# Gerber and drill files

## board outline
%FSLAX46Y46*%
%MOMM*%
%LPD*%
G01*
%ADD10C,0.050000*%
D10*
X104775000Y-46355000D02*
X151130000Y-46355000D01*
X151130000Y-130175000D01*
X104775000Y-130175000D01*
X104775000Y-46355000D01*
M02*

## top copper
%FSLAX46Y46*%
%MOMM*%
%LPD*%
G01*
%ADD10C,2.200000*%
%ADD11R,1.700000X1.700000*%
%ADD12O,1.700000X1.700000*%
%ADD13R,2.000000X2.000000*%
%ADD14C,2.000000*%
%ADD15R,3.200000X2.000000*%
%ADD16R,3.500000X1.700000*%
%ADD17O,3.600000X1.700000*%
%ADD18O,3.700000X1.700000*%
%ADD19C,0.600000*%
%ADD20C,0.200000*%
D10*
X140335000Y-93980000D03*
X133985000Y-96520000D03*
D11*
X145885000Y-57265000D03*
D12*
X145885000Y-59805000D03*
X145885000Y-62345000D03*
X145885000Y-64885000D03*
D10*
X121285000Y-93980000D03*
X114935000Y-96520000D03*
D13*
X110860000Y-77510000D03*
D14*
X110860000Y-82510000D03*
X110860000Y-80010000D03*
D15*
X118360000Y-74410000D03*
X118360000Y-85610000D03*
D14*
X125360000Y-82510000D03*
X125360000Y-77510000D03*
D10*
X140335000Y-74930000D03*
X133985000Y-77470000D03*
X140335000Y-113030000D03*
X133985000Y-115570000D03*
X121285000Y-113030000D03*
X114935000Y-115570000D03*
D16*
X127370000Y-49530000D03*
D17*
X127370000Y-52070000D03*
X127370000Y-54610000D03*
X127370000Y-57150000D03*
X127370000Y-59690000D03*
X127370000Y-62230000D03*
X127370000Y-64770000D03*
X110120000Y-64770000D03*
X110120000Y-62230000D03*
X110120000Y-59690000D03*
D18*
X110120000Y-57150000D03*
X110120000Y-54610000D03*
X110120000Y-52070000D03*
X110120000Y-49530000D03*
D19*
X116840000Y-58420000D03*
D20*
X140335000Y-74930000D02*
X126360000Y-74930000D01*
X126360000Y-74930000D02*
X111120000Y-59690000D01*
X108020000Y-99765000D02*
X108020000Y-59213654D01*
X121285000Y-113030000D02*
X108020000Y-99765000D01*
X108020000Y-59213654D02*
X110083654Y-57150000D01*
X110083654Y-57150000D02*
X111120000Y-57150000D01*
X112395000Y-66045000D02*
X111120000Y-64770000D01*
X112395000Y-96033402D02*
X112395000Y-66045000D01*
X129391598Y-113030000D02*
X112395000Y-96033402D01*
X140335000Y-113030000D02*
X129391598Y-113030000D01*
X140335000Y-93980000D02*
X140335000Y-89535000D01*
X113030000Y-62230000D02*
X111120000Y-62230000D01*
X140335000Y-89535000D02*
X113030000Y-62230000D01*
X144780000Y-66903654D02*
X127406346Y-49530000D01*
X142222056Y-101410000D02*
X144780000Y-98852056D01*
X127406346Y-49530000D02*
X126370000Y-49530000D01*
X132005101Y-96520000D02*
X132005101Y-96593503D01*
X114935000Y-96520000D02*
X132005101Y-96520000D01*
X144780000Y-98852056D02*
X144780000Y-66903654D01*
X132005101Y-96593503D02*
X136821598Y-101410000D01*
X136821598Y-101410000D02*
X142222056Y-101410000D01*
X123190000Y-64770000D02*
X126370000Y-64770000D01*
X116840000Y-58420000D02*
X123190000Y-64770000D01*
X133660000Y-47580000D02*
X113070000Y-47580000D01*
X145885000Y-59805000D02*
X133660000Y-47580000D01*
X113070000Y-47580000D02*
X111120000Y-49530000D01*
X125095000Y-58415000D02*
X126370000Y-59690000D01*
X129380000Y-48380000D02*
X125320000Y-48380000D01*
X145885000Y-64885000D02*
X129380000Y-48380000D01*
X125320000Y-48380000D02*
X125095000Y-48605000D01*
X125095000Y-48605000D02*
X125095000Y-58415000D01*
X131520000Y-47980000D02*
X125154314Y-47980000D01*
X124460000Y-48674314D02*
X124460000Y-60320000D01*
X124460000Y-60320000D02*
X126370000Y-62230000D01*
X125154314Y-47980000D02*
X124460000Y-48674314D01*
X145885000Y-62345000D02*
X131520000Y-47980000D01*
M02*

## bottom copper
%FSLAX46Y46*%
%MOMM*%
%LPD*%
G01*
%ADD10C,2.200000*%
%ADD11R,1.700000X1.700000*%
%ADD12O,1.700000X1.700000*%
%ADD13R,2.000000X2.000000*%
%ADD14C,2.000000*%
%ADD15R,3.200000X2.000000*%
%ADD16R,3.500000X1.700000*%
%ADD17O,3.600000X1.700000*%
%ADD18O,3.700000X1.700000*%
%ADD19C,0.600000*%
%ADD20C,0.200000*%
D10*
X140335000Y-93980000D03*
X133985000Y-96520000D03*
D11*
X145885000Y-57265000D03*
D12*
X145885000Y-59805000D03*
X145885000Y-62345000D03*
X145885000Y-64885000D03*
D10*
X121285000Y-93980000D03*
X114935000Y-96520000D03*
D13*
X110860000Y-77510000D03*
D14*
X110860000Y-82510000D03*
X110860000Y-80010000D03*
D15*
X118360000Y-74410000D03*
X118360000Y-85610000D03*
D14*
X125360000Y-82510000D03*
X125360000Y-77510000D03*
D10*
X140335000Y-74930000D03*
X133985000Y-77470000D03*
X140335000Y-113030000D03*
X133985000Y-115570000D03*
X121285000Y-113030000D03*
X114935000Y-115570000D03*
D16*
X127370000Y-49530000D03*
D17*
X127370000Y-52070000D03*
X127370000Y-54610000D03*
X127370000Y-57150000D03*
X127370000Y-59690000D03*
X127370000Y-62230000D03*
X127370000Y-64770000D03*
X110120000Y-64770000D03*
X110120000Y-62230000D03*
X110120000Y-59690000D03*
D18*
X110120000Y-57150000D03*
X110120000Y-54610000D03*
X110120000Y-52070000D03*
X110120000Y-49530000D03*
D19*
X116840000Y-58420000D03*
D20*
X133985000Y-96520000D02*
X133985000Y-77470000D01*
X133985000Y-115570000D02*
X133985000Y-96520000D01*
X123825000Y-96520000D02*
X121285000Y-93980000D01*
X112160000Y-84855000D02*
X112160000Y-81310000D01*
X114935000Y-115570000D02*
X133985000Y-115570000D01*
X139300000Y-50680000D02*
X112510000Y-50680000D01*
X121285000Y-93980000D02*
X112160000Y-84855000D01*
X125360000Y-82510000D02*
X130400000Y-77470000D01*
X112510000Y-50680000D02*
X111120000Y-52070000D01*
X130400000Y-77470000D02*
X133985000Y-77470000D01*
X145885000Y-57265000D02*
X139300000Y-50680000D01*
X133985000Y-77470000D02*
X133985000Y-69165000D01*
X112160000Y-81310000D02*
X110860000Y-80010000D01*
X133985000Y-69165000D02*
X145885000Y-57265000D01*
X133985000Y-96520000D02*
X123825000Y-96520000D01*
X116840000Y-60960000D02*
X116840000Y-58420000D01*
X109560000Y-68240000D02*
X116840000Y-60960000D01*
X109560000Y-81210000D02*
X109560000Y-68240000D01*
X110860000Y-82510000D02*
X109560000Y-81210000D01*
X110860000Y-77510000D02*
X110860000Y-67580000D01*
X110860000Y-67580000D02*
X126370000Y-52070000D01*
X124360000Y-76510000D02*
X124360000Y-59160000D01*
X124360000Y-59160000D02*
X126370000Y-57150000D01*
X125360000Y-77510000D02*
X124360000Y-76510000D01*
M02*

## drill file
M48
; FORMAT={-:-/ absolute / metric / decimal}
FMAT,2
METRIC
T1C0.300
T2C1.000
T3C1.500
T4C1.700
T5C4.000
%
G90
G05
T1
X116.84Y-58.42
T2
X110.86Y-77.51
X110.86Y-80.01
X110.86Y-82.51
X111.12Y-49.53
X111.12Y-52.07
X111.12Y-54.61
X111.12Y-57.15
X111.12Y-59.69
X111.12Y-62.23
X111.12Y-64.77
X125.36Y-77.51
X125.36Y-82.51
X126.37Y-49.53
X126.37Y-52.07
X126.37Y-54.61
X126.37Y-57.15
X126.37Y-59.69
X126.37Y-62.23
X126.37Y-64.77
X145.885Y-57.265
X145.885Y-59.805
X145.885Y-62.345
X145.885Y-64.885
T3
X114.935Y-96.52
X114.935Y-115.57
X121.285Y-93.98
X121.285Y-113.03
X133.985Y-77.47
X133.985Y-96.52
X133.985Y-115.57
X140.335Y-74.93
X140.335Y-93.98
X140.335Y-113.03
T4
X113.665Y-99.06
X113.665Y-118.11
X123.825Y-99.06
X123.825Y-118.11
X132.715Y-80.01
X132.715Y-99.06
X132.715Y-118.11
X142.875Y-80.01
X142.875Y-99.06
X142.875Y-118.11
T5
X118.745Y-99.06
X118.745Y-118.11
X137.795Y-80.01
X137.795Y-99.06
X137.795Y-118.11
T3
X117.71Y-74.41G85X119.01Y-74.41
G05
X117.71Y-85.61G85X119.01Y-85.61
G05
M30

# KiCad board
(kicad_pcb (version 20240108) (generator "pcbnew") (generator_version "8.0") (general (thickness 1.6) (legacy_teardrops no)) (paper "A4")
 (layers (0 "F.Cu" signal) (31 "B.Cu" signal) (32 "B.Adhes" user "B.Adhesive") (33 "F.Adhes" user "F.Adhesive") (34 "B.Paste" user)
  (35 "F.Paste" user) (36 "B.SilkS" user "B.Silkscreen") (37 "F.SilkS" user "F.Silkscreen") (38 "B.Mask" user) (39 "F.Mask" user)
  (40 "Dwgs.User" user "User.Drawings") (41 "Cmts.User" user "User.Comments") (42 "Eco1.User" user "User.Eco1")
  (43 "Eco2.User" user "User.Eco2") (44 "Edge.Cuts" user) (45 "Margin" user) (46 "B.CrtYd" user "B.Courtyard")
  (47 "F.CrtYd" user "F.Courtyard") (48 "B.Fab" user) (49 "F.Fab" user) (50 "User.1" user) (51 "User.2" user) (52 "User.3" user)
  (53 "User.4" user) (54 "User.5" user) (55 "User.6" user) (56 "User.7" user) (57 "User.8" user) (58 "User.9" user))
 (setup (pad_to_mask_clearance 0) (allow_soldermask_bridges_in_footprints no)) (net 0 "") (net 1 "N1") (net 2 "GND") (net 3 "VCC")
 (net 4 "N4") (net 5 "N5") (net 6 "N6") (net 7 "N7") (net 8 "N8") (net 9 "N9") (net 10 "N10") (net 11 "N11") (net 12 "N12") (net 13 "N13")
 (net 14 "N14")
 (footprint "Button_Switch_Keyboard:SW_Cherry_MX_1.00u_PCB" (layer "F.Cu") (at 140.335 93.98)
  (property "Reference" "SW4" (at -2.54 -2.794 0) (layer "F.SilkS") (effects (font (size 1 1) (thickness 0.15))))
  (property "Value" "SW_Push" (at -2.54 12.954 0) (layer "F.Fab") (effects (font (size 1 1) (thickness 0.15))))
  (pad "" np_thru_hole circle (at -7.62 5.08) (size 1.7 1.7) (drill 1.7) (layers "*.Cu" "*.Mask"))
  (pad "" np_thru_hole circle (at -2.54 5.08) (size 4 4) (drill 4) (layers "*.Cu" "*.Mask"))
  (pad "" np_thru_hole circle (at 2.54 5.08) (size 1.7 1.7) (drill 1.7) (layers "*.Cu" "*.Mask"))
  (pad "1" thru_hole circle (at 0 0) (size 2.2 2.2) (drill 1.5) (layers "*.Cu" "*.Mask") (remove_unused_layers no) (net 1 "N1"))
  (pad "2" thru_hole circle (at -6.35 2.54) (size 2.2 2.2) (drill 1.5) (layers "*.Cu" "*.Mask") (remove_unused_layers no) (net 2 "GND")))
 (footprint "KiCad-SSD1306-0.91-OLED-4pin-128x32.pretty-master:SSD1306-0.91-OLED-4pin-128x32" (layer "F.Cu") (at 109.385 55.075)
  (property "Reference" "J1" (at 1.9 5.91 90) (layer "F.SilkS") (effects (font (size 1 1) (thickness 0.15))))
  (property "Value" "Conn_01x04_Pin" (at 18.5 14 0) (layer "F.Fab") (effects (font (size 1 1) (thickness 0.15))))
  (pad "1" thru_hole rect (at 36.5 2.19) (size 1.7 1.7) (drill 1) (layers "*.Cu" "*.Mask") (remove_unused_layers no) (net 2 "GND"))
  (pad "2" thru_hole oval (at 36.5 4.73) (size 1.7 1.7) (drill 1) (layers "*.Cu" "*.Mask") (remove_unused_layers no) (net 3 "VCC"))
  (pad "3" thru_hole oval (at 36.5 7.27) (size 1.7 1.7) (drill 1) (layers "*.Cu" "*.Mask") (remove_unused_layers no) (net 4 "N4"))
  (pad "4" thru_hole oval (at 36.5 9.81) (size 1.7 1.7) (drill 1) (layers "*.Cu" "*.Mask") (remove_unused_layers no) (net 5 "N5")))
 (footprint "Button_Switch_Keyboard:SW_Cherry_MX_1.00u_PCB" (layer "F.Cu") (at 121.285 93.98)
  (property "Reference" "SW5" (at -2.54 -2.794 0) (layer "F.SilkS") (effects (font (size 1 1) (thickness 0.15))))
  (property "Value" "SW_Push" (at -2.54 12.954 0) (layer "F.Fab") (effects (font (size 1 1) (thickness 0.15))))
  (pad "" np_thru_hole circle (at -7.62 5.08) (size 1.7 1.7) (drill 1.7) (layers "*.Cu" "*.Mask"))
  (pad "" np_thru_hole circle (at -2.54 5.08) (size 4 4) (drill 4) (layers "*.Cu" "*.Mask"))
  (pad "" np_thru_hole circle (at 2.54 5.08) (size 1.7 1.7) (drill 1.7) (layers "*.Cu" "*.Mask"))
  (pad "1" thru_hole circle (at 0 0) (size 2.2 2.2) (drill 1.5) (layers "*.Cu" "*.Mask") (remove_unused_layers no) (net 2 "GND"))
  (pad "2" thru_hole circle (at -6.35 2.54) (size 2.2 2.2) (drill 1.5) (layers "*.Cu" "*.Mask") (remove_unused_layers no) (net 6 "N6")))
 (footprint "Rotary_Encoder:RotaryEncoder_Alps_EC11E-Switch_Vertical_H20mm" (layer "F.Cu") (at 110.86 77.51)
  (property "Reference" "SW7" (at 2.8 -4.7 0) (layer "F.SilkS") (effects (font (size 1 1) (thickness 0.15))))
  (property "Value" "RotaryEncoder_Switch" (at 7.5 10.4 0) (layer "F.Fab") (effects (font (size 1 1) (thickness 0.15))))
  (pad "A" thru_hole rect (at 0 0) (size 2 2) (drill 1) (layers "*.Cu" "*.Mask") (remove_unused_layers no) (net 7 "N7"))
  (pad "B" thru_hole circle (at 0 5) (size 2 2) (drill 1) (layers "*.Cu" "*.Mask") (remove_unused_layers no) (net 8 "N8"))
  (pad "C" thru_hole circle (at 0 2.5) (size 2 2) (drill 1) (layers "*.Cu" "*.Mask") (remove_unused_layers no) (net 2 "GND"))
  (pad "MP" thru_hole rect (at 7.5 -3.1) (size 3.2 2) (drill oval 2.8 1.5) (layers "*.Cu" "*.Mask") (remove_unused_layers no))
  (pad "MP" thru_hole rect (at 7.5 8.1) (size 3.2 2) (drill oval 2.8 1.5) (layers "*.Cu" "*.Mask") (remove_unused_layers no))
  (pad "S1" thru_hole circle (at 14.5 5) (size 2 2) (drill 1) (layers "*.Cu" "*.Mask") (remove_unused_layers no) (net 2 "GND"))
  (pad "S2" thru_hole circle (at 14.5 0) (size 2 2) (drill 1) (layers "*.Cu" "*.Mask") (remove_unused_layers no) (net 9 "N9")))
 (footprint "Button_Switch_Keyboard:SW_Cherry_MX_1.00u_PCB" (layer "F.Cu") (at 140.335 74.93)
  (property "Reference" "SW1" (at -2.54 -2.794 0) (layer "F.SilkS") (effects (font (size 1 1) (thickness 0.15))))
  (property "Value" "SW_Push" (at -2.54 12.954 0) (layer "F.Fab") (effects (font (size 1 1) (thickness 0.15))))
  (pad "" np_thru_hole circle (at -7.62 5.08) (size 1.7 1.7) (drill 1.7) (layers "*.Cu" "*.Mask"))
  (pad "" np_thru_hole circle (at -2.54 5.08) (size 4 4) (drill 4) (layers "*.Cu" "*.Mask"))
  (pad "" np_thru_hole circle (at 2.54 5.08) (size 1.7 1.7) (drill 1.7) (layers "*.Cu" "*.Mask"))
  (pad "1" thru_hole circle (at 0 0) (size 2.2 2.2) (drill 1.5) (layers "*.Cu" "*.Mask") (remove_unused_layers no) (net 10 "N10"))
  (pad "2" thru_hole circle (at -6.35 2.54) (size 2.2 2.2) (drill 1.5) (layers "*.Cu" "*.Mask") (remove_unused_layers no) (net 2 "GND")))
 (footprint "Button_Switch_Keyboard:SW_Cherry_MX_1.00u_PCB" (layer "F.Cu") (at 140.335 113.03)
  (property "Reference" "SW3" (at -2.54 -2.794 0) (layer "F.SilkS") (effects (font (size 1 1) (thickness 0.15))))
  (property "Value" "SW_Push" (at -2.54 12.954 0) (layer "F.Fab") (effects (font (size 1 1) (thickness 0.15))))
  (pad "" np_thru_hole circle (at -7.62 5.08) (size 1.7 1.7) (drill 1.7) (layers "*.Cu" "*.Mask"))
  (pad "" np_thru_hole circle (at -2.54 5.08) (size 4 4) (drill 4) (layers "*.Cu" "*.Mask"))
  (pad "" np_thru_hole circle (at 2.54 5.08) (size 1.7 1.7) (drill 1.7) (layers "*.Cu" "*.Mask"))
  (pad "1" thru_hole circle (at 0 0) (size 2.2 2.2) (drill 1.5) (layers "*.Cu" "*.Mask") (remove_unused_layers no) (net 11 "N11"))
  (pad "2" thru_hole circle (at -6.35 2.54) (size 2.2 2.2) (drill 1.5) (layers "*.Cu" "*.Mask") (remove_unused_layers no) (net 2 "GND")))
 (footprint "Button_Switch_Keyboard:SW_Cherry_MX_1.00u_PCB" (layer "F.Cu") (at 121.285 113.03)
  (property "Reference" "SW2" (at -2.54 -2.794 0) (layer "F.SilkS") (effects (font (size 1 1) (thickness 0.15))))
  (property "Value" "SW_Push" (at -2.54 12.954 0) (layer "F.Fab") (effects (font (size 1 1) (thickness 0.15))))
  (pad "" np_thru_hole circle (at -7.62 5.08) (size 1.7 1.7) (drill 1.7) (layers "*.Cu" "*.Mask"))
  (pad "" np_thru_hole circle (at -2.54 5.08) (size 4 4) (drill 4) (layers "*.Cu" "*.Mask"))
  (pad "" np_thru_hole circle (at 2.54 5.08) (size 1.7 1.7) (drill 1.7) (layers "*.Cu" "*.Mask"))
  (pad "1" thru_hole circle (at 0 0) (size 2.2 2.2) (drill 1.5) (layers "*.Cu" "*.Mask") (remove_unused_layers no) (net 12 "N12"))
  (pad "2" thru_hole circle (at -6.35 2.54) (size 2.2 2.2) (drill 1.5) (layers "*.Cu" "*.Mask") (remove_unused_layers no) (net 2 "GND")))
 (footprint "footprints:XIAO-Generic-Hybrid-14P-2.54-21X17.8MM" (layer "B.Cu") (at 118.745 57.15 180)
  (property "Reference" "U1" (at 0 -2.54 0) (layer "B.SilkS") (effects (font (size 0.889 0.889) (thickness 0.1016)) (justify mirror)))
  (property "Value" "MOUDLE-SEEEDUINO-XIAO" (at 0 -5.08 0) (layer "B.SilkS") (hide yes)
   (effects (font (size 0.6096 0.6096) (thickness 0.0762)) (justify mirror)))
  (pad "1" thru_hole rect (at -7.625 7.62 180) (size 3.5 1.7) (drill 1 (offset -1 0)) (layers "*.Cu" "*.Mask") (remove_unused_layers no)
   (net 6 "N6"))
  (pad "2" thru_hole oval (at -7.625 5.08 180) (size 3.6 1.7) (drill 1 (offset -1 0)) (layers "*.Cu" "*.Mask") (remove_unused_layers no)
   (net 7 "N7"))
  (pad "3" thru_hole oval (at -7.625 2.54 180) (size 3.6 1.7) (drill 1 (offset -1 0)) (layers "*.Cu" "*.Mask") (remove_unused_layers no)
   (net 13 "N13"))
  (pad "4" thru_hole oval (at -7.625 0 180) (size 3.6 1.7) (drill 1 (offset -1 0)) (layers "*.Cu" "*.Mask") (remove_unused_layers no)
   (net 9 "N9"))
  (pad "5" thru_hole oval (at -7.625 -2.54 180) (size 3.6 1.7) (drill 1 (offset -1 0)) (layers "*.Cu" "*.Mask") (remove_unused_layers no)
   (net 5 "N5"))
  (pad "6" thru_hole oval (at -7.625 -5.08) (size 3.6 1.7) (drill 1 (offset 1 0)) (layers "*.Cu" "*.Mask") (remove_unused_layers no)
   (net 4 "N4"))
  (pad "7" thru_hole oval (at -7.625 -7.62 180) (size 3.6 1.7) (drill 1 (offset -1 0)) (layers "*.Cu" "*.Mask") (remove_unused_layers no)
   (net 8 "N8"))
  (pad "8" thru_hole oval (at 7.625 -7.62 180) (size 3.6 1.7) (drill 1 (offset 1 0)) (layers "*.Cu" "*.Mask") (remove_unused_layers no)
   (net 11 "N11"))
  (pad "9" thru_hole oval (at 7.625 -5.08 180) (size 3.6 1.7) (drill 1 (offset 1 0)) (layers "*.Cu" "*.Mask") (remove_unused_layers no)
   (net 1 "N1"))
  (pad "10" thru_hole oval (at 7.625 -2.54 180) (size 3.6 1.7) (drill 1 (offset 1 0)) (layers "*.Cu" "*.Mask") (remove_unused_layers no)
   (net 10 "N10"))
  (pad "11" thru_hole oval (at 7.625 0 180) (size 3.7 1.7) (drill 1 (offset 1 0)) (layers "*.Cu" "*.Mask") (remove_unused_layers no)
   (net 12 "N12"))
  (pad "12" thru_hole oval (at 7.625 2.54 180) (size 3.7 1.7) (drill 1 (offset 1 0)) (layers "*.Cu" "*.Mask") (remove_unused_layers no)
   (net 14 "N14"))
  (pad "13" thru_hole oval (at 7.625 5.08 180) (size 3.7 1.7) (drill 1 (offset 1 0)) (layers "*.Cu" "*.Mask") (remove_unused_layers no)
   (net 2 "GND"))
  (pad "14" thru_hole oval (at 7.625 7.62 180) (size 3.7 1.7) (drill 1 (offset 1 0)) (layers "*.Cu" "*.Mask") (remove_unused_layers no)
   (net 3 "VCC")))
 (gr_rect (start 104.775 46.355) (end 151.13 130.175) (stroke (width 0.05) (type default)) (fill none) (layer "Edge.Cuts"))
 (segment (start 133.985 96.52) (end 133.985 77.47) (width 0.2) (layer "B.Cu") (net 2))
 (segment (start 133.985 115.57) (end 133.985 96.52) (width 0.2) (layer "B.Cu") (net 2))
 (segment (start 123.825 96.52) (end 121.285 93.98) (width 0.2) (layer "B.Cu") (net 2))
 (segment (start 112.16 84.855) (end 112.16 81.31) (width 0.2) (layer "B.Cu") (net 2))
 (segment (start 114.935 115.57) (end 133.985 115.57) (width 0.2) (layer "B.Cu") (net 2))
 (segment (start 139.3 50.68) (end 112.51 50.68) (width 0.2) (layer "B.Cu") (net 2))
 (segment (start 121.285 93.98) (end 112.16 84.855) (width 0.2) (layer "B.Cu") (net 2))
 (segment (start 125.36 82.51) (end 130.4 77.47) (width 0.2) (layer "B.Cu") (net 2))
 (segment (start 112.51 50.68) (end 111.12 52.07) (width 0.2) (layer "B.Cu") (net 2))
 (segment (start 130.4 77.47) (end 133.985 77.47) (width 0.2) (layer "B.Cu") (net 2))
 (segment (start 145.885 57.265) (end 139.3 50.68) (width 0.2) (layer "B.Cu") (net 2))
 (segment (start 133.985 77.47) (end 133.985 69.165) (width 0.2) (layer "B.Cu") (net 2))
 (segment (start 112.16 81.31) (end 110.86 80.01) (width 0.2) (layer "B.Cu") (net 2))
 (segment (start 133.985 69.165) (end 145.885 57.265) (width 0.2) (layer "B.Cu") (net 2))
 (segment (start 133.985 96.52) (end 123.825 96.52) (width 0.2) (layer "B.Cu") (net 2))
 (segment (start 140.335 74.93) (end 126.36 74.93) (width 0.2) (layer "F.Cu") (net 10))
 (segment (start 126.36 74.93) (end 111.12 59.69) (width 0.2) (layer "F.Cu") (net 10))
 (segment (start 108.02 99.765) (end 108.02 59.213654) (width 0.2) (layer "F.Cu") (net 12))
 (segment (start 121.285 113.03) (end 108.02 99.765) (width 0.2) (layer "F.Cu") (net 12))
 (segment (start 108.02 59.213654) (end 110.083654 57.15) (width 0.2) (layer "F.Cu") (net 12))
 (segment (start 110.083654 57.15) (end 111.12 57.15) (width 0.2) (layer "F.Cu") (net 12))
 (segment (start 112.395 66.045) (end 111.12 64.77) (width 0.2) (layer "F.Cu") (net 11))
 (segment (start 112.395 96.033402) (end 112.395 66.045) (width 0.2) (layer "F.Cu") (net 11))
 (segment (start 129.391598 113.03) (end 112.395 96.033402) (width 0.2) (layer "F.Cu") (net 11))
 (segment (start 140.335 113.03) (end 129.391598 113.03) (width 0.2) (layer "F.Cu") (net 11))
 (segment (start 140.335 93.98) (end 140.335 89.535) (width 0.2) (layer "F.Cu") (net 1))
 (segment (start 113.03 62.23) (end 111.12 62.23) (width 0.2) (layer "F.Cu") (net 1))
 (segment (start 140.335 89.535) (end 113.03 62.23) (width 0.2) (layer "F.Cu") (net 1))
 (segment (start 144.78 66.903654) (end 127.406346 49.53) (width 0.2) (layer "F.Cu") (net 6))
 (segment (start 142.222056 101.41) (end 144.78 98.852056) (width 0.2) (layer "F.Cu") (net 6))
 (segment (start 127.406346 49.53) (end 126.37 49.53) (width 0.2) (layer "F.Cu") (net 6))
 (segment (start 132.005101 96.52) (end 132.005101 96.593503) (width 0.2) (layer "F.Cu") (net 6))
 (segment (start 114.935 96.52) (end 132.005101 96.52) (width 0.2) (layer "F.Cu") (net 6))
 (segment (start 144.78 98.852056) (end 144.78 66.903654) (width 0.2) (layer "F.Cu") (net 6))
 (segment (start 132.005101 96.593503) (end 136.821598 101.41) (width 0.2) (layer "F.Cu") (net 6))
 (segment (start 136.821598 101.41) (end 142.222056 101.41) (width 0.2) (layer "F.Cu") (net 6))
 (segment (start 123.19 64.77) (end 126.37 64.77) (width 0.2) (layer "F.Cu") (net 8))
 (segment (start 116.84 58.42) (end 123.19 64.77) (width 0.2) (layer "F.Cu") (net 8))
 (via (at 116.84 58.42) (size 0.6) (drill 0.3) (layers "F.Cu" "B.Cu") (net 8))
 (segment (start 116.84 60.96) (end 116.84 58.42) (width 0.2) (layer "B.Cu") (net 8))
 (segment (start 109.56 68.24) (end 116.84 60.96) (width 0.2) (layer "B.Cu") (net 8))
 (segment (start 109.56 81.21) (end 109.56 68.24) (width 0.2) (layer "B.Cu") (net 8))
 (segment (start 110.86 82.51) (end 109.56 81.21) (width 0.2) (layer "B.Cu") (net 8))
 (segment (start 110.86 77.51) (end 110.86 67.58) (width 0.2) (layer "B.Cu") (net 7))
 (segment (start 110.86 67.58) (end 126.37 52.07) (width 0.2) (layer "B.Cu") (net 7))
 (segment (start 124.36 76.51) (end 124.36 59.16) (width 0.2) (layer "B.Cu") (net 9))
 (segment (start 124.36 59.16) (end 126.37 57.15) (width 0.2) (layer "B.Cu") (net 9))
 (segment (start 125.36 77.51) (end 124.36 76.51) (width 0.2) (layer "B.Cu") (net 9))
 (segment (start 133.66 47.58) (end 113.07 47.58) (width 0.2) (layer "F.Cu") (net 3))
 (segment (start 145.885 59.805) (end 133.66 47.58) (width 0.2) (layer "F.Cu") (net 3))
 (segment (start 113.07 47.58) (end 111.12 49.53) (width 0.2) (layer "F.Cu") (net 3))
 (segment (start 125.095 58.415) (end 126.37 59.69) (width 0.2) (layer "F.Cu") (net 5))
 (segment (start 129.38 48.38) (end 125.32 48.38) (width 0.2) (layer "F.Cu") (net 5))
 (segment (start 145.885 64.885) (end 129.38 48.38) (width 0.2) (layer "F.Cu") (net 5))
 (segment (start 125.32 48.38) (end 125.095 48.605) (width 0.2) (layer "F.Cu") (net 5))
 (segment (start 125.095 48.605) (end 125.095 58.415) (width 0.2) (layer "F.Cu") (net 5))
 (segment (start 131.52 47.98) (end 125.154314 47.98) (width 0.2) (layer "F.Cu") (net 4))
 (segment (start 124.46 48.674314) (end 124.46 60.32) (width 0.2) (layer "F.Cu") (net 4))
 (segment (start 124.46 60.32) (end 126.37 62.23) (width 0.2) (layer "F.Cu") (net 4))
 (segment (start 125.154314 47.98) (end 124.46 48.674314) (width 0.2) (layer "F.Cu") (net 4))
 (segment (start 145.885 62.345) (end 131.52 47.98) (width 0.2) (layer "F.Cu") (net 4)))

